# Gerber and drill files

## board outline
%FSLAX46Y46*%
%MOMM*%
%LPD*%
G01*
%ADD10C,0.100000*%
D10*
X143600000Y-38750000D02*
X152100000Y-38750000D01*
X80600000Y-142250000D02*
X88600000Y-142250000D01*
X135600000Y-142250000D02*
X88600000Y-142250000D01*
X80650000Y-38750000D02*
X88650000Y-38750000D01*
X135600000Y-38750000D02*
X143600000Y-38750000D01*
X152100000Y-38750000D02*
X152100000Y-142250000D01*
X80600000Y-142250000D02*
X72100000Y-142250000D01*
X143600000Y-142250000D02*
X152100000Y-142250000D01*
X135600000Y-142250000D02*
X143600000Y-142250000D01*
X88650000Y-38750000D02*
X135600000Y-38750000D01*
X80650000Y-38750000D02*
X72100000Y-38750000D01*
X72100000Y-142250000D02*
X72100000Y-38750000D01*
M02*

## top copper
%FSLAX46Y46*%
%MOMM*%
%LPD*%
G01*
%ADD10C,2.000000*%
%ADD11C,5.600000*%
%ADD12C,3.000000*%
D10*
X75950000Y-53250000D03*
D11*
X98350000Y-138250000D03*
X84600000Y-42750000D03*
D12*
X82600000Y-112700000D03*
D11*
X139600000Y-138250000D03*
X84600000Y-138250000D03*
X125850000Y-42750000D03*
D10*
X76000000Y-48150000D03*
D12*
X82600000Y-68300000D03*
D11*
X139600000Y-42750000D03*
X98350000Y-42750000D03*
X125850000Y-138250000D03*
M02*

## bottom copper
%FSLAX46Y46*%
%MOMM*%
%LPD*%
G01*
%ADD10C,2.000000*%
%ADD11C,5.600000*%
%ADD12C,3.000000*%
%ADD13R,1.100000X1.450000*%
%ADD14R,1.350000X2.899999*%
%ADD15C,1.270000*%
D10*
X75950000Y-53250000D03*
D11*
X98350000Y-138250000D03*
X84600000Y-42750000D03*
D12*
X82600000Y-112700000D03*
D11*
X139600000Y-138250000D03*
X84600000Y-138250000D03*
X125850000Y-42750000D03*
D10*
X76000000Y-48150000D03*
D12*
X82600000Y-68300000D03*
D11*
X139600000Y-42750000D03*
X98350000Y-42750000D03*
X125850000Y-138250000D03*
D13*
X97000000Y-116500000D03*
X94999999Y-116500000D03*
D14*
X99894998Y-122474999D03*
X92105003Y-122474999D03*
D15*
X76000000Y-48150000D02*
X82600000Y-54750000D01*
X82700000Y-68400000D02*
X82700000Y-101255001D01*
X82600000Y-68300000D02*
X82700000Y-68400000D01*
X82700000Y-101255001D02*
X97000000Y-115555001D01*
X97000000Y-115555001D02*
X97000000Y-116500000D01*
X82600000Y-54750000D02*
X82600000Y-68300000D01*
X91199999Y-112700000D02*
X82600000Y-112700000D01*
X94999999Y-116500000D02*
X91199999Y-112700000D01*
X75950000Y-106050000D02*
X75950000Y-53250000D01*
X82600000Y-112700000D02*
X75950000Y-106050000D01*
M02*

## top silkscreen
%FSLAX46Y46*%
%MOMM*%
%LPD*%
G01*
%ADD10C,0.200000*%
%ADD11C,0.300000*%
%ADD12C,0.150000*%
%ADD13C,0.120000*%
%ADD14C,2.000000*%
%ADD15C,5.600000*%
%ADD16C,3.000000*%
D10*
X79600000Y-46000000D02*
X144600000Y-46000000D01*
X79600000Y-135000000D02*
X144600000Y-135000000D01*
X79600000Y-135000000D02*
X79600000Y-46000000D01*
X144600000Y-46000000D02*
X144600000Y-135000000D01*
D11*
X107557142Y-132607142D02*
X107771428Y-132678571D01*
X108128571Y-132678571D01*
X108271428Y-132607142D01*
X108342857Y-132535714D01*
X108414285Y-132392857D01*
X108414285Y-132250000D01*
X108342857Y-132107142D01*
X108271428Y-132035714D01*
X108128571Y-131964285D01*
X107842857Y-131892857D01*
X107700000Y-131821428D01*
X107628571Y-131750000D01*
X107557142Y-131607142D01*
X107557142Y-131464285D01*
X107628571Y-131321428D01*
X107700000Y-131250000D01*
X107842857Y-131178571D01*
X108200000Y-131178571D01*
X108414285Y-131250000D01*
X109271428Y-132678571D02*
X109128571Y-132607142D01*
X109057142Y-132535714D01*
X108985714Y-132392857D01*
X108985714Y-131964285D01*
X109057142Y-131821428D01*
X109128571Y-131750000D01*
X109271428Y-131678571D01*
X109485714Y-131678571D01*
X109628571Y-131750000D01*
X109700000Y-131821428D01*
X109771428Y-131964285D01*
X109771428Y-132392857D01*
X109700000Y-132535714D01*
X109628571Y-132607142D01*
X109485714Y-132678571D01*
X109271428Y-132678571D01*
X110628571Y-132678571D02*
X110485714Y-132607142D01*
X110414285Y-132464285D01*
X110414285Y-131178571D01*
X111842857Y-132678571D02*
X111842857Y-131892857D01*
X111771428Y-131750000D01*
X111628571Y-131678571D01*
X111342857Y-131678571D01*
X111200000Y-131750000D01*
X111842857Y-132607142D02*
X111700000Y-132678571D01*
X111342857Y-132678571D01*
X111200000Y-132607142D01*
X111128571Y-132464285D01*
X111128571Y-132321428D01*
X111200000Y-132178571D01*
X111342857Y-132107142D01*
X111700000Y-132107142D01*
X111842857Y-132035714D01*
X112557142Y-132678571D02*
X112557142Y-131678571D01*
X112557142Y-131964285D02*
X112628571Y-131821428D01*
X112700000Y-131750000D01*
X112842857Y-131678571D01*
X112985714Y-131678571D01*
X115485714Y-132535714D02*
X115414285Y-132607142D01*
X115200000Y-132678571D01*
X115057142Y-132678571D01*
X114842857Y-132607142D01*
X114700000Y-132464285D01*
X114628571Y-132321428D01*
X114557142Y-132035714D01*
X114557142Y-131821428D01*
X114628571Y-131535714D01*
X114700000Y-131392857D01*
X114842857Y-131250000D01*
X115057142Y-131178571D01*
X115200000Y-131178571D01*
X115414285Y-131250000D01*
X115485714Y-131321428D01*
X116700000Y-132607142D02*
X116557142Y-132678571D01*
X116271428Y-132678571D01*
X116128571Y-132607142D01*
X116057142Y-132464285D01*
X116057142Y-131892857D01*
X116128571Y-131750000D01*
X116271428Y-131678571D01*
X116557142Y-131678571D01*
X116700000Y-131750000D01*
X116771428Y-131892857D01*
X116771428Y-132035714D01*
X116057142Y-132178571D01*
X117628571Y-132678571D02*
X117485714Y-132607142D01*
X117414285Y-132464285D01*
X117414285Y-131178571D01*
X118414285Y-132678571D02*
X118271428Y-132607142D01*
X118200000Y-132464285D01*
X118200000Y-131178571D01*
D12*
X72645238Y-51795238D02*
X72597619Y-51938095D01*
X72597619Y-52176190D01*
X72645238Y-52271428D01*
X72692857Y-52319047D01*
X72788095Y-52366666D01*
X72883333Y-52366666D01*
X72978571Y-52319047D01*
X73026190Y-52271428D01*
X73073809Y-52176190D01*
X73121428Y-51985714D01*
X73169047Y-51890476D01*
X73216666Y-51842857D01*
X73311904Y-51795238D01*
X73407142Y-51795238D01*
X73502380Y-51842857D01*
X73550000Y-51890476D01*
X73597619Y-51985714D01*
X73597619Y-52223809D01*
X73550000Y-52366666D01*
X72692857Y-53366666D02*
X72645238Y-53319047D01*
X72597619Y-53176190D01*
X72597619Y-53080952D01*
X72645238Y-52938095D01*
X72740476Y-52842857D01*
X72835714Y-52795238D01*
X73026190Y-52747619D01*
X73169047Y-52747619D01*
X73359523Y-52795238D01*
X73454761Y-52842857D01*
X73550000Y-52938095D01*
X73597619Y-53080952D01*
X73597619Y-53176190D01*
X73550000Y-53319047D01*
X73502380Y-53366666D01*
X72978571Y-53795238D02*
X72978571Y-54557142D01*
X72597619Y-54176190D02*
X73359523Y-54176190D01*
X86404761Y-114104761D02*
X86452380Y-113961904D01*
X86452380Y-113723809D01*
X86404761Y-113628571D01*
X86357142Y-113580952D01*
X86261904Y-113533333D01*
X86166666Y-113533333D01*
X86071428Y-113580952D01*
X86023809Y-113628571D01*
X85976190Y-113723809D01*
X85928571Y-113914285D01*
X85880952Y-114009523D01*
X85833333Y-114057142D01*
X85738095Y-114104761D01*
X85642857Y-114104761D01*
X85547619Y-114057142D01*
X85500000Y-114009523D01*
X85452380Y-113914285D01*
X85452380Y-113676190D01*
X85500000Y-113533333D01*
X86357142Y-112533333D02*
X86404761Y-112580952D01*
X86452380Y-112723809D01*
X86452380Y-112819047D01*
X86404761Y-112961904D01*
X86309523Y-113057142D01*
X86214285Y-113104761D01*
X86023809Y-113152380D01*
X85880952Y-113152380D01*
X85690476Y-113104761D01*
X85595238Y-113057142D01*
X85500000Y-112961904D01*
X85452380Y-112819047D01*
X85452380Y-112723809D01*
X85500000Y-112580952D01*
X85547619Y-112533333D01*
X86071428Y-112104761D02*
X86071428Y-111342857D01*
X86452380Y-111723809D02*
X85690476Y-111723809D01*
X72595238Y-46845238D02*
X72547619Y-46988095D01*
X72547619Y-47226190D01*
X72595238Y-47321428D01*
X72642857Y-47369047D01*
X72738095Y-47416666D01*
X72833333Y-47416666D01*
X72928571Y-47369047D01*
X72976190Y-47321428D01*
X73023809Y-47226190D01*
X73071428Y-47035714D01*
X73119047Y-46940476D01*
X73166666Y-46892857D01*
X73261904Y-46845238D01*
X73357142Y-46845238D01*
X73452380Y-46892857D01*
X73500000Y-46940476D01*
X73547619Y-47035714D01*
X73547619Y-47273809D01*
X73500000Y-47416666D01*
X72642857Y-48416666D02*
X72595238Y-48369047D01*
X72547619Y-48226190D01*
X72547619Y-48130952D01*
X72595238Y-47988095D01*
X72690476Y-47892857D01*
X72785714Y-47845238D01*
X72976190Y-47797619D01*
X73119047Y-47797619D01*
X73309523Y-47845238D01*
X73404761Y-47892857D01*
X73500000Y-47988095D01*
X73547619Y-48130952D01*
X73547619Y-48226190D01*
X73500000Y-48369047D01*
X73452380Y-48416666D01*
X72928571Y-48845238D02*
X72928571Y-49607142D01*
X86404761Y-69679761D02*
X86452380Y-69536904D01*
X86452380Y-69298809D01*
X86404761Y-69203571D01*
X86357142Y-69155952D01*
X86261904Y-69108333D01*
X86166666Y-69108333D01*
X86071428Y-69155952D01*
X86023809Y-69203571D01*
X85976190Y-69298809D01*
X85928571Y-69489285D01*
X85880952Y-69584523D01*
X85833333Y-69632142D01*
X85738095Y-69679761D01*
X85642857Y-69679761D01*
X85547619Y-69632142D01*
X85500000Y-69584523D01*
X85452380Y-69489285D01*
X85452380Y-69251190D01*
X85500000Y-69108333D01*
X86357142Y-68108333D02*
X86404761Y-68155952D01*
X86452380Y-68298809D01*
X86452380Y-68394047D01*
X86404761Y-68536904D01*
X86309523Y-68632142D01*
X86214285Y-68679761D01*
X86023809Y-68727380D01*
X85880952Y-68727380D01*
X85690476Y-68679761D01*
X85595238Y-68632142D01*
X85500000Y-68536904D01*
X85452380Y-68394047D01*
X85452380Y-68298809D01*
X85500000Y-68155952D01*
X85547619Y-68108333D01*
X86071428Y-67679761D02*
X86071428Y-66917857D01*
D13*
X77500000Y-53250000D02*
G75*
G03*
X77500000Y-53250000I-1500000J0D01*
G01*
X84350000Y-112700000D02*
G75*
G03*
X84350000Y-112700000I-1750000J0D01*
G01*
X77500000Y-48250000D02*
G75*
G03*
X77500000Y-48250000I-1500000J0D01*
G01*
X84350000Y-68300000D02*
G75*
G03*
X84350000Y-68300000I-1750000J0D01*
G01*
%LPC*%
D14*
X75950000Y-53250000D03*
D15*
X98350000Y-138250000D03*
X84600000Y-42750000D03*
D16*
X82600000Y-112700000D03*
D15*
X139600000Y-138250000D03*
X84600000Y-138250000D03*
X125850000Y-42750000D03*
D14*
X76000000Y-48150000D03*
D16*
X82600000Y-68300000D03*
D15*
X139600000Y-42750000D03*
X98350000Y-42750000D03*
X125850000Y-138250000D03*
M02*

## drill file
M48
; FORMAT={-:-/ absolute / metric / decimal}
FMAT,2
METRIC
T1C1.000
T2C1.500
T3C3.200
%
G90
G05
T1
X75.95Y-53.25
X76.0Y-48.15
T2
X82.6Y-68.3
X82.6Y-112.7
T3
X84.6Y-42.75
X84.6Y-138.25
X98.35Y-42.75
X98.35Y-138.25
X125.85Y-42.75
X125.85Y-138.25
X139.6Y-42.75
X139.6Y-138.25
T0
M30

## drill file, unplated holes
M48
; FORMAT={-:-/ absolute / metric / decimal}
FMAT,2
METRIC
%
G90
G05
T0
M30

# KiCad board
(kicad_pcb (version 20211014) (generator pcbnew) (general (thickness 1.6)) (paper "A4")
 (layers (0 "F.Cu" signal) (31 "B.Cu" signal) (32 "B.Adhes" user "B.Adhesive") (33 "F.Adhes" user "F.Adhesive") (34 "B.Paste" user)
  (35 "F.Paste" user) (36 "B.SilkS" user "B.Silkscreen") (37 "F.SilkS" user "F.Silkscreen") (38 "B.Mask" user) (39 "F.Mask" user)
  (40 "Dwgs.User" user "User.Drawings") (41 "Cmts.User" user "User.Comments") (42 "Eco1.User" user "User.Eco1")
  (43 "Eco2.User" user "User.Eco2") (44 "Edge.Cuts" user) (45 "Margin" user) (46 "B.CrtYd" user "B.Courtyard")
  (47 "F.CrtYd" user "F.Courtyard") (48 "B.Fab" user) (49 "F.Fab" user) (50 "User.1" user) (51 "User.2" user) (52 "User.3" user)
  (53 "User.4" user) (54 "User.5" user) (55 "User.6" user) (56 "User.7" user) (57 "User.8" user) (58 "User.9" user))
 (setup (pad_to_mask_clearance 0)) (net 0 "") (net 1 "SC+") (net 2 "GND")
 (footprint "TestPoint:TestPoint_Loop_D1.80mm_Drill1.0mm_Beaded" (layer "F.Cu") (at 76 53.25)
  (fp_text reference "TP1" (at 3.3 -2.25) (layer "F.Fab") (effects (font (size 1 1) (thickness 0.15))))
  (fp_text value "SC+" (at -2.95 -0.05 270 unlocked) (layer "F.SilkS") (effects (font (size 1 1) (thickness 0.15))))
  (fp_circle (center 0 0) (end 1.5 0) (layer "F.SilkS") (width 0.12) (fill none))
  (pad "1" thru_hole circle (at -0.05 0) (size 2 2) (drill 1) (layers *.Cu *.Mask) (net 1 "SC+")))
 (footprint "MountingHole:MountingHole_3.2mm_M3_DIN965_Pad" (layer "F.Cu") (at 98.35 138.25)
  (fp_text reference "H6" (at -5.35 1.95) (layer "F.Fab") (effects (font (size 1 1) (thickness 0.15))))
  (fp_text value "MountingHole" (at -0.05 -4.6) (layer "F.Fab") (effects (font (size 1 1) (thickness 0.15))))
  (pad "1" thru_hole circle (at 0 0) (size 5.6 5.6) (drill 3.2) (layers *.Cu *.Mask)))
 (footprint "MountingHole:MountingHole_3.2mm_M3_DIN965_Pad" (layer "F.Cu") (at 84.6 42.75)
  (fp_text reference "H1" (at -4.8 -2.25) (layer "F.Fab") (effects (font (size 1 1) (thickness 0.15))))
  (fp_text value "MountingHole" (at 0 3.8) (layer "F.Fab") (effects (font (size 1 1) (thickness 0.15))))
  (pad "1" thru_hole circle (at 0 0) (size 5.6 5.6) (drill 3.2) (layers *.Cu *.Mask)))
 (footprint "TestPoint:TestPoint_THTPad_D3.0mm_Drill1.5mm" (layer "F.Cu") (at 82.6 112.7)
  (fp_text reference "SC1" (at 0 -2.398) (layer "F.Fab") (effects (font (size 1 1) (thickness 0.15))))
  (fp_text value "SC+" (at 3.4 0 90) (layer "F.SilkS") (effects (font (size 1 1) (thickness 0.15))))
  (fp_circle (center 0 0) (end 0 1.75) (layer "F.SilkS") (width 0.12) (fill none))
  (pad "1" thru_hole circle (at 0 0) (size 3 3) (drill 1.5) (layers *.Cu *.Mask) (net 1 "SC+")))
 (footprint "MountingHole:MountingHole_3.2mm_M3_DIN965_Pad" (layer "F.Cu") (at 139.6 138.25)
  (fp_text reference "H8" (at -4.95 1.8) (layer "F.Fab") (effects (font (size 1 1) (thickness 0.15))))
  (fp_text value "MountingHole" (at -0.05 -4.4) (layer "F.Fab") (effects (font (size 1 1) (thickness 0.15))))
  (pad "1" thru_hole circle (at 0 0) (size 5.6 5.6) (drill 3.2) (layers *.Cu *.Mask)))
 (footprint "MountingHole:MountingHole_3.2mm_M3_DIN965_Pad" (layer "F.Cu") (at 84.6 138.25)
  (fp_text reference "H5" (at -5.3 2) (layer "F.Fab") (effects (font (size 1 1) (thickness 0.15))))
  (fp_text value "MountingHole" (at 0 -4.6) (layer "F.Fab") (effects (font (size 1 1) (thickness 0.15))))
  (pad "1" thru_hole circle (at 0 0) (size 5.6 5.6) (drill 3.2) (layers *.Cu *.Mask)))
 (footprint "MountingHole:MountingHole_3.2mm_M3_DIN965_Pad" (layer "F.Cu") (at 125.85 42.75)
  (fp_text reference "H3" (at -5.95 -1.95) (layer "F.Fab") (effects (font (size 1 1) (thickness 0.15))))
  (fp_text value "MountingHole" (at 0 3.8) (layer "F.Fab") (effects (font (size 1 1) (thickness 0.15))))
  (pad "1" thru_hole circle (at 0 0) (size 5.6 5.6) (drill 3.2) (layers *.Cu *.Mask)))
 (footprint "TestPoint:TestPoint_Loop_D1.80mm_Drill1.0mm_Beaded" (layer "F.Cu") (at 76 48.25)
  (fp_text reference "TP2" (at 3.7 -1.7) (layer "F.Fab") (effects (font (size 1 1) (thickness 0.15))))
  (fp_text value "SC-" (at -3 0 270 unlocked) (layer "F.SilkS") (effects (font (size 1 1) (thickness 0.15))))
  (fp_circle (center 0 0) (end 1.5 0) (layer "F.SilkS") (width 0.12) (fill none))
  (pad "1" thru_hole circle (at 0 -0.1) (size 2 2) (drill 1) (layers *.Cu *.Mask) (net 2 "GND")))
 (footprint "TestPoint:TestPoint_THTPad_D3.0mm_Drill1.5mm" (layer "F.Cu") (at 82.6 68.3)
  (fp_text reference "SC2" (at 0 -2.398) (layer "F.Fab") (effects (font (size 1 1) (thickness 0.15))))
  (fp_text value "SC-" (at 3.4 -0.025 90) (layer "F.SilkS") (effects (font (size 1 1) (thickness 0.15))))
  (fp_circle (center 0 0) (end 0 1.75) (layer "F.SilkS") (width 0.12) (fill none))
  (pad "1" thru_hole circle (at 0 0) (size 3 3) (drill 1.5) (layers *.Cu *.Mask) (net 2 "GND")))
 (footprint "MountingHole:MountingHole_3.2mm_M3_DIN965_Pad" (layer "F.Cu") (at 139.6 42.75)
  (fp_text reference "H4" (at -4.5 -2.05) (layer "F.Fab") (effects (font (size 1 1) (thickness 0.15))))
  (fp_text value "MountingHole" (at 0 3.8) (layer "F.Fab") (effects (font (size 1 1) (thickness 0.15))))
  (pad "1" thru_hole circle (at 0 0) (size 5.6 5.6) (drill 3.2) (layers *.Cu *.Mask)))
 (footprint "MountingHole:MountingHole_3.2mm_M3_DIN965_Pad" (layer "F.Cu") (at 98.35 42.75)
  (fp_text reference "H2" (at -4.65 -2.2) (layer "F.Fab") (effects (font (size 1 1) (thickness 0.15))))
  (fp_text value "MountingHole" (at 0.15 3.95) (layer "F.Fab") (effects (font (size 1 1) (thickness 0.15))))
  (pad "1" thru_hole circle (at 0 0) (size 5.6 5.6) (drill 3.2) (layers *.Cu *.Mask)))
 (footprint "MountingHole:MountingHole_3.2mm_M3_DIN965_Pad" (layer "F.Cu") (at 125.85 138.25)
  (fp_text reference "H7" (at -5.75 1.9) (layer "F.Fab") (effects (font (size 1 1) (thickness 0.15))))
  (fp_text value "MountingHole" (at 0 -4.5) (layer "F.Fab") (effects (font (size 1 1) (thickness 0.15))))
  (pad "1" thru_hole circle (at 0 0) (size 5.6 5.6) (drill 3.2) (layers *.Cu *.Mask)))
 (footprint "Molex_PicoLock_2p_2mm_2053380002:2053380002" (layer "B.Cu") (at 97 116.5)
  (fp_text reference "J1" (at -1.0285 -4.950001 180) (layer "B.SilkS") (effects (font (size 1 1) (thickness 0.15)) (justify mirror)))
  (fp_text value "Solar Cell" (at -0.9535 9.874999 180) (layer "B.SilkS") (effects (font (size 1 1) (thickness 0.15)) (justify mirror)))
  (pad "1" smd rect (at 0 0) (size 1.1 1.45) (layers "B.Cu" "B.Paste" "B.Mask") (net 2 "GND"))
  (pad "2" smd rect (at -2.000001 0) (size 1.1 1.45) (layers "B.Cu" "B.Paste" "B.Mask") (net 1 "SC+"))
  (pad "3" smd rect (at 2.894998 5.974999) (size 1.35 2.899999) (layers "B.Cu" "B.Paste" "B.Mask"))
  (pad "4" smd rect (at -4.894997 5.974999) (size 1.35 2.899999) (layers "B.Cu" "B.Paste" "B.Mask")))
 (gr_line (start 79.6 46) (end 144.6 46) (layer "F.SilkS") (width 0.2))
 (gr_line (start 79.6 135) (end 144.6 135) (layer "F.SilkS") (width 0.2))
 (gr_line (start 79.6 135) (end 79.6 46) (layer "F.SilkS") (width 0.2))
 (gr_line (start 144.6 46) (end 144.6 135) (layer "F.SilkS") (width 0.2))
 (gr_line (start 143.6 38.75) (end 152.1 38.75) (layer "Edge.Cuts") (width 0.1))
 (gr_line (start 80.6 142.25) (end 88.6 142.25) (layer "Edge.Cuts") (width 0.1))
 (gr_line (start 135.6 142.25) (end 88.6 142.25) (layer "Edge.Cuts") (width 0.1))
 (gr_line (start 80.65 38.75) (end 88.65 38.75) (layer "Edge.Cuts") (width 0.1))
 (gr_line (start 135.6 38.75) (end 143.6 38.75) (layer "Edge.Cuts") (width 0.1))
 (gr_line (start 152.1 38.75) (end 152.1 142.25) (layer "Edge.Cuts") (width 0.1))
 (gr_line (start 80.6 142.25) (end 72.1 142.25) (layer "Edge.Cuts") (width 0.1))
 (gr_line (start 143.6 142.25) (end 152.1 142.25) (layer "Edge.Cuts") (width 0.1))
 (gr_line (start 135.6 142.25) (end 143.6 142.25) (layer "Edge.Cuts") (width 0.1))
 (gr_line (start 88.65 38.75) (end 135.6 38.75) (layer "Edge.Cuts") (width 0.1))
 (gr_line (start 80.65 38.75) (end 72.1 38.75) (layer "Edge.Cuts") (width 0.1))
 (gr_line (start 72.1 142.25) (end 72.1 38.75) (layer "Edge.Cuts") (width 0.1))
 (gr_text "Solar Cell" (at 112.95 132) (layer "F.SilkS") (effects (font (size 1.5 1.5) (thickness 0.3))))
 (segment (start 76 48.15) (end 82.6 54.75) (width 1.27) (layer "B.Cu") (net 2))
 (segment (start 82.7 68.4) (end 82.7 101.255001) (width 1.27) (layer "B.Cu") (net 2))
 (segment (start 82.6 68.3) (end 82.7 68.4) (width 1.27) (layer "B.Cu") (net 2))
 (segment (start 82.7 101.255001) (end 97 115.555001) (width 1.27) (layer "B.Cu") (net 2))
 (segment (start 97 115.555001) (end 97 116.5) (width 1.27) (layer "B.Cu") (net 2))
 (segment (start 82.6 54.75) (end 82.6 68.3) (width 1.27) (layer "B.Cu") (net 2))
 (segment (start 91.199999 112.7) (end 82.6 112.7) (width 1.27) (layer "B.Cu") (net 1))
 (segment (start 94.999999 116.5) (end 91.199999 112.7) (width 1.27) (layer "B.Cu") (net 1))
 (segment (start 75.95 106.05) (end 75.95 53.25) (width 1.27) (layer "B.Cu") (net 1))
 (segment (start 82.6 112.7) (end 75.95 106.05) (width 1.27) (layer "B.Cu") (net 1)))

